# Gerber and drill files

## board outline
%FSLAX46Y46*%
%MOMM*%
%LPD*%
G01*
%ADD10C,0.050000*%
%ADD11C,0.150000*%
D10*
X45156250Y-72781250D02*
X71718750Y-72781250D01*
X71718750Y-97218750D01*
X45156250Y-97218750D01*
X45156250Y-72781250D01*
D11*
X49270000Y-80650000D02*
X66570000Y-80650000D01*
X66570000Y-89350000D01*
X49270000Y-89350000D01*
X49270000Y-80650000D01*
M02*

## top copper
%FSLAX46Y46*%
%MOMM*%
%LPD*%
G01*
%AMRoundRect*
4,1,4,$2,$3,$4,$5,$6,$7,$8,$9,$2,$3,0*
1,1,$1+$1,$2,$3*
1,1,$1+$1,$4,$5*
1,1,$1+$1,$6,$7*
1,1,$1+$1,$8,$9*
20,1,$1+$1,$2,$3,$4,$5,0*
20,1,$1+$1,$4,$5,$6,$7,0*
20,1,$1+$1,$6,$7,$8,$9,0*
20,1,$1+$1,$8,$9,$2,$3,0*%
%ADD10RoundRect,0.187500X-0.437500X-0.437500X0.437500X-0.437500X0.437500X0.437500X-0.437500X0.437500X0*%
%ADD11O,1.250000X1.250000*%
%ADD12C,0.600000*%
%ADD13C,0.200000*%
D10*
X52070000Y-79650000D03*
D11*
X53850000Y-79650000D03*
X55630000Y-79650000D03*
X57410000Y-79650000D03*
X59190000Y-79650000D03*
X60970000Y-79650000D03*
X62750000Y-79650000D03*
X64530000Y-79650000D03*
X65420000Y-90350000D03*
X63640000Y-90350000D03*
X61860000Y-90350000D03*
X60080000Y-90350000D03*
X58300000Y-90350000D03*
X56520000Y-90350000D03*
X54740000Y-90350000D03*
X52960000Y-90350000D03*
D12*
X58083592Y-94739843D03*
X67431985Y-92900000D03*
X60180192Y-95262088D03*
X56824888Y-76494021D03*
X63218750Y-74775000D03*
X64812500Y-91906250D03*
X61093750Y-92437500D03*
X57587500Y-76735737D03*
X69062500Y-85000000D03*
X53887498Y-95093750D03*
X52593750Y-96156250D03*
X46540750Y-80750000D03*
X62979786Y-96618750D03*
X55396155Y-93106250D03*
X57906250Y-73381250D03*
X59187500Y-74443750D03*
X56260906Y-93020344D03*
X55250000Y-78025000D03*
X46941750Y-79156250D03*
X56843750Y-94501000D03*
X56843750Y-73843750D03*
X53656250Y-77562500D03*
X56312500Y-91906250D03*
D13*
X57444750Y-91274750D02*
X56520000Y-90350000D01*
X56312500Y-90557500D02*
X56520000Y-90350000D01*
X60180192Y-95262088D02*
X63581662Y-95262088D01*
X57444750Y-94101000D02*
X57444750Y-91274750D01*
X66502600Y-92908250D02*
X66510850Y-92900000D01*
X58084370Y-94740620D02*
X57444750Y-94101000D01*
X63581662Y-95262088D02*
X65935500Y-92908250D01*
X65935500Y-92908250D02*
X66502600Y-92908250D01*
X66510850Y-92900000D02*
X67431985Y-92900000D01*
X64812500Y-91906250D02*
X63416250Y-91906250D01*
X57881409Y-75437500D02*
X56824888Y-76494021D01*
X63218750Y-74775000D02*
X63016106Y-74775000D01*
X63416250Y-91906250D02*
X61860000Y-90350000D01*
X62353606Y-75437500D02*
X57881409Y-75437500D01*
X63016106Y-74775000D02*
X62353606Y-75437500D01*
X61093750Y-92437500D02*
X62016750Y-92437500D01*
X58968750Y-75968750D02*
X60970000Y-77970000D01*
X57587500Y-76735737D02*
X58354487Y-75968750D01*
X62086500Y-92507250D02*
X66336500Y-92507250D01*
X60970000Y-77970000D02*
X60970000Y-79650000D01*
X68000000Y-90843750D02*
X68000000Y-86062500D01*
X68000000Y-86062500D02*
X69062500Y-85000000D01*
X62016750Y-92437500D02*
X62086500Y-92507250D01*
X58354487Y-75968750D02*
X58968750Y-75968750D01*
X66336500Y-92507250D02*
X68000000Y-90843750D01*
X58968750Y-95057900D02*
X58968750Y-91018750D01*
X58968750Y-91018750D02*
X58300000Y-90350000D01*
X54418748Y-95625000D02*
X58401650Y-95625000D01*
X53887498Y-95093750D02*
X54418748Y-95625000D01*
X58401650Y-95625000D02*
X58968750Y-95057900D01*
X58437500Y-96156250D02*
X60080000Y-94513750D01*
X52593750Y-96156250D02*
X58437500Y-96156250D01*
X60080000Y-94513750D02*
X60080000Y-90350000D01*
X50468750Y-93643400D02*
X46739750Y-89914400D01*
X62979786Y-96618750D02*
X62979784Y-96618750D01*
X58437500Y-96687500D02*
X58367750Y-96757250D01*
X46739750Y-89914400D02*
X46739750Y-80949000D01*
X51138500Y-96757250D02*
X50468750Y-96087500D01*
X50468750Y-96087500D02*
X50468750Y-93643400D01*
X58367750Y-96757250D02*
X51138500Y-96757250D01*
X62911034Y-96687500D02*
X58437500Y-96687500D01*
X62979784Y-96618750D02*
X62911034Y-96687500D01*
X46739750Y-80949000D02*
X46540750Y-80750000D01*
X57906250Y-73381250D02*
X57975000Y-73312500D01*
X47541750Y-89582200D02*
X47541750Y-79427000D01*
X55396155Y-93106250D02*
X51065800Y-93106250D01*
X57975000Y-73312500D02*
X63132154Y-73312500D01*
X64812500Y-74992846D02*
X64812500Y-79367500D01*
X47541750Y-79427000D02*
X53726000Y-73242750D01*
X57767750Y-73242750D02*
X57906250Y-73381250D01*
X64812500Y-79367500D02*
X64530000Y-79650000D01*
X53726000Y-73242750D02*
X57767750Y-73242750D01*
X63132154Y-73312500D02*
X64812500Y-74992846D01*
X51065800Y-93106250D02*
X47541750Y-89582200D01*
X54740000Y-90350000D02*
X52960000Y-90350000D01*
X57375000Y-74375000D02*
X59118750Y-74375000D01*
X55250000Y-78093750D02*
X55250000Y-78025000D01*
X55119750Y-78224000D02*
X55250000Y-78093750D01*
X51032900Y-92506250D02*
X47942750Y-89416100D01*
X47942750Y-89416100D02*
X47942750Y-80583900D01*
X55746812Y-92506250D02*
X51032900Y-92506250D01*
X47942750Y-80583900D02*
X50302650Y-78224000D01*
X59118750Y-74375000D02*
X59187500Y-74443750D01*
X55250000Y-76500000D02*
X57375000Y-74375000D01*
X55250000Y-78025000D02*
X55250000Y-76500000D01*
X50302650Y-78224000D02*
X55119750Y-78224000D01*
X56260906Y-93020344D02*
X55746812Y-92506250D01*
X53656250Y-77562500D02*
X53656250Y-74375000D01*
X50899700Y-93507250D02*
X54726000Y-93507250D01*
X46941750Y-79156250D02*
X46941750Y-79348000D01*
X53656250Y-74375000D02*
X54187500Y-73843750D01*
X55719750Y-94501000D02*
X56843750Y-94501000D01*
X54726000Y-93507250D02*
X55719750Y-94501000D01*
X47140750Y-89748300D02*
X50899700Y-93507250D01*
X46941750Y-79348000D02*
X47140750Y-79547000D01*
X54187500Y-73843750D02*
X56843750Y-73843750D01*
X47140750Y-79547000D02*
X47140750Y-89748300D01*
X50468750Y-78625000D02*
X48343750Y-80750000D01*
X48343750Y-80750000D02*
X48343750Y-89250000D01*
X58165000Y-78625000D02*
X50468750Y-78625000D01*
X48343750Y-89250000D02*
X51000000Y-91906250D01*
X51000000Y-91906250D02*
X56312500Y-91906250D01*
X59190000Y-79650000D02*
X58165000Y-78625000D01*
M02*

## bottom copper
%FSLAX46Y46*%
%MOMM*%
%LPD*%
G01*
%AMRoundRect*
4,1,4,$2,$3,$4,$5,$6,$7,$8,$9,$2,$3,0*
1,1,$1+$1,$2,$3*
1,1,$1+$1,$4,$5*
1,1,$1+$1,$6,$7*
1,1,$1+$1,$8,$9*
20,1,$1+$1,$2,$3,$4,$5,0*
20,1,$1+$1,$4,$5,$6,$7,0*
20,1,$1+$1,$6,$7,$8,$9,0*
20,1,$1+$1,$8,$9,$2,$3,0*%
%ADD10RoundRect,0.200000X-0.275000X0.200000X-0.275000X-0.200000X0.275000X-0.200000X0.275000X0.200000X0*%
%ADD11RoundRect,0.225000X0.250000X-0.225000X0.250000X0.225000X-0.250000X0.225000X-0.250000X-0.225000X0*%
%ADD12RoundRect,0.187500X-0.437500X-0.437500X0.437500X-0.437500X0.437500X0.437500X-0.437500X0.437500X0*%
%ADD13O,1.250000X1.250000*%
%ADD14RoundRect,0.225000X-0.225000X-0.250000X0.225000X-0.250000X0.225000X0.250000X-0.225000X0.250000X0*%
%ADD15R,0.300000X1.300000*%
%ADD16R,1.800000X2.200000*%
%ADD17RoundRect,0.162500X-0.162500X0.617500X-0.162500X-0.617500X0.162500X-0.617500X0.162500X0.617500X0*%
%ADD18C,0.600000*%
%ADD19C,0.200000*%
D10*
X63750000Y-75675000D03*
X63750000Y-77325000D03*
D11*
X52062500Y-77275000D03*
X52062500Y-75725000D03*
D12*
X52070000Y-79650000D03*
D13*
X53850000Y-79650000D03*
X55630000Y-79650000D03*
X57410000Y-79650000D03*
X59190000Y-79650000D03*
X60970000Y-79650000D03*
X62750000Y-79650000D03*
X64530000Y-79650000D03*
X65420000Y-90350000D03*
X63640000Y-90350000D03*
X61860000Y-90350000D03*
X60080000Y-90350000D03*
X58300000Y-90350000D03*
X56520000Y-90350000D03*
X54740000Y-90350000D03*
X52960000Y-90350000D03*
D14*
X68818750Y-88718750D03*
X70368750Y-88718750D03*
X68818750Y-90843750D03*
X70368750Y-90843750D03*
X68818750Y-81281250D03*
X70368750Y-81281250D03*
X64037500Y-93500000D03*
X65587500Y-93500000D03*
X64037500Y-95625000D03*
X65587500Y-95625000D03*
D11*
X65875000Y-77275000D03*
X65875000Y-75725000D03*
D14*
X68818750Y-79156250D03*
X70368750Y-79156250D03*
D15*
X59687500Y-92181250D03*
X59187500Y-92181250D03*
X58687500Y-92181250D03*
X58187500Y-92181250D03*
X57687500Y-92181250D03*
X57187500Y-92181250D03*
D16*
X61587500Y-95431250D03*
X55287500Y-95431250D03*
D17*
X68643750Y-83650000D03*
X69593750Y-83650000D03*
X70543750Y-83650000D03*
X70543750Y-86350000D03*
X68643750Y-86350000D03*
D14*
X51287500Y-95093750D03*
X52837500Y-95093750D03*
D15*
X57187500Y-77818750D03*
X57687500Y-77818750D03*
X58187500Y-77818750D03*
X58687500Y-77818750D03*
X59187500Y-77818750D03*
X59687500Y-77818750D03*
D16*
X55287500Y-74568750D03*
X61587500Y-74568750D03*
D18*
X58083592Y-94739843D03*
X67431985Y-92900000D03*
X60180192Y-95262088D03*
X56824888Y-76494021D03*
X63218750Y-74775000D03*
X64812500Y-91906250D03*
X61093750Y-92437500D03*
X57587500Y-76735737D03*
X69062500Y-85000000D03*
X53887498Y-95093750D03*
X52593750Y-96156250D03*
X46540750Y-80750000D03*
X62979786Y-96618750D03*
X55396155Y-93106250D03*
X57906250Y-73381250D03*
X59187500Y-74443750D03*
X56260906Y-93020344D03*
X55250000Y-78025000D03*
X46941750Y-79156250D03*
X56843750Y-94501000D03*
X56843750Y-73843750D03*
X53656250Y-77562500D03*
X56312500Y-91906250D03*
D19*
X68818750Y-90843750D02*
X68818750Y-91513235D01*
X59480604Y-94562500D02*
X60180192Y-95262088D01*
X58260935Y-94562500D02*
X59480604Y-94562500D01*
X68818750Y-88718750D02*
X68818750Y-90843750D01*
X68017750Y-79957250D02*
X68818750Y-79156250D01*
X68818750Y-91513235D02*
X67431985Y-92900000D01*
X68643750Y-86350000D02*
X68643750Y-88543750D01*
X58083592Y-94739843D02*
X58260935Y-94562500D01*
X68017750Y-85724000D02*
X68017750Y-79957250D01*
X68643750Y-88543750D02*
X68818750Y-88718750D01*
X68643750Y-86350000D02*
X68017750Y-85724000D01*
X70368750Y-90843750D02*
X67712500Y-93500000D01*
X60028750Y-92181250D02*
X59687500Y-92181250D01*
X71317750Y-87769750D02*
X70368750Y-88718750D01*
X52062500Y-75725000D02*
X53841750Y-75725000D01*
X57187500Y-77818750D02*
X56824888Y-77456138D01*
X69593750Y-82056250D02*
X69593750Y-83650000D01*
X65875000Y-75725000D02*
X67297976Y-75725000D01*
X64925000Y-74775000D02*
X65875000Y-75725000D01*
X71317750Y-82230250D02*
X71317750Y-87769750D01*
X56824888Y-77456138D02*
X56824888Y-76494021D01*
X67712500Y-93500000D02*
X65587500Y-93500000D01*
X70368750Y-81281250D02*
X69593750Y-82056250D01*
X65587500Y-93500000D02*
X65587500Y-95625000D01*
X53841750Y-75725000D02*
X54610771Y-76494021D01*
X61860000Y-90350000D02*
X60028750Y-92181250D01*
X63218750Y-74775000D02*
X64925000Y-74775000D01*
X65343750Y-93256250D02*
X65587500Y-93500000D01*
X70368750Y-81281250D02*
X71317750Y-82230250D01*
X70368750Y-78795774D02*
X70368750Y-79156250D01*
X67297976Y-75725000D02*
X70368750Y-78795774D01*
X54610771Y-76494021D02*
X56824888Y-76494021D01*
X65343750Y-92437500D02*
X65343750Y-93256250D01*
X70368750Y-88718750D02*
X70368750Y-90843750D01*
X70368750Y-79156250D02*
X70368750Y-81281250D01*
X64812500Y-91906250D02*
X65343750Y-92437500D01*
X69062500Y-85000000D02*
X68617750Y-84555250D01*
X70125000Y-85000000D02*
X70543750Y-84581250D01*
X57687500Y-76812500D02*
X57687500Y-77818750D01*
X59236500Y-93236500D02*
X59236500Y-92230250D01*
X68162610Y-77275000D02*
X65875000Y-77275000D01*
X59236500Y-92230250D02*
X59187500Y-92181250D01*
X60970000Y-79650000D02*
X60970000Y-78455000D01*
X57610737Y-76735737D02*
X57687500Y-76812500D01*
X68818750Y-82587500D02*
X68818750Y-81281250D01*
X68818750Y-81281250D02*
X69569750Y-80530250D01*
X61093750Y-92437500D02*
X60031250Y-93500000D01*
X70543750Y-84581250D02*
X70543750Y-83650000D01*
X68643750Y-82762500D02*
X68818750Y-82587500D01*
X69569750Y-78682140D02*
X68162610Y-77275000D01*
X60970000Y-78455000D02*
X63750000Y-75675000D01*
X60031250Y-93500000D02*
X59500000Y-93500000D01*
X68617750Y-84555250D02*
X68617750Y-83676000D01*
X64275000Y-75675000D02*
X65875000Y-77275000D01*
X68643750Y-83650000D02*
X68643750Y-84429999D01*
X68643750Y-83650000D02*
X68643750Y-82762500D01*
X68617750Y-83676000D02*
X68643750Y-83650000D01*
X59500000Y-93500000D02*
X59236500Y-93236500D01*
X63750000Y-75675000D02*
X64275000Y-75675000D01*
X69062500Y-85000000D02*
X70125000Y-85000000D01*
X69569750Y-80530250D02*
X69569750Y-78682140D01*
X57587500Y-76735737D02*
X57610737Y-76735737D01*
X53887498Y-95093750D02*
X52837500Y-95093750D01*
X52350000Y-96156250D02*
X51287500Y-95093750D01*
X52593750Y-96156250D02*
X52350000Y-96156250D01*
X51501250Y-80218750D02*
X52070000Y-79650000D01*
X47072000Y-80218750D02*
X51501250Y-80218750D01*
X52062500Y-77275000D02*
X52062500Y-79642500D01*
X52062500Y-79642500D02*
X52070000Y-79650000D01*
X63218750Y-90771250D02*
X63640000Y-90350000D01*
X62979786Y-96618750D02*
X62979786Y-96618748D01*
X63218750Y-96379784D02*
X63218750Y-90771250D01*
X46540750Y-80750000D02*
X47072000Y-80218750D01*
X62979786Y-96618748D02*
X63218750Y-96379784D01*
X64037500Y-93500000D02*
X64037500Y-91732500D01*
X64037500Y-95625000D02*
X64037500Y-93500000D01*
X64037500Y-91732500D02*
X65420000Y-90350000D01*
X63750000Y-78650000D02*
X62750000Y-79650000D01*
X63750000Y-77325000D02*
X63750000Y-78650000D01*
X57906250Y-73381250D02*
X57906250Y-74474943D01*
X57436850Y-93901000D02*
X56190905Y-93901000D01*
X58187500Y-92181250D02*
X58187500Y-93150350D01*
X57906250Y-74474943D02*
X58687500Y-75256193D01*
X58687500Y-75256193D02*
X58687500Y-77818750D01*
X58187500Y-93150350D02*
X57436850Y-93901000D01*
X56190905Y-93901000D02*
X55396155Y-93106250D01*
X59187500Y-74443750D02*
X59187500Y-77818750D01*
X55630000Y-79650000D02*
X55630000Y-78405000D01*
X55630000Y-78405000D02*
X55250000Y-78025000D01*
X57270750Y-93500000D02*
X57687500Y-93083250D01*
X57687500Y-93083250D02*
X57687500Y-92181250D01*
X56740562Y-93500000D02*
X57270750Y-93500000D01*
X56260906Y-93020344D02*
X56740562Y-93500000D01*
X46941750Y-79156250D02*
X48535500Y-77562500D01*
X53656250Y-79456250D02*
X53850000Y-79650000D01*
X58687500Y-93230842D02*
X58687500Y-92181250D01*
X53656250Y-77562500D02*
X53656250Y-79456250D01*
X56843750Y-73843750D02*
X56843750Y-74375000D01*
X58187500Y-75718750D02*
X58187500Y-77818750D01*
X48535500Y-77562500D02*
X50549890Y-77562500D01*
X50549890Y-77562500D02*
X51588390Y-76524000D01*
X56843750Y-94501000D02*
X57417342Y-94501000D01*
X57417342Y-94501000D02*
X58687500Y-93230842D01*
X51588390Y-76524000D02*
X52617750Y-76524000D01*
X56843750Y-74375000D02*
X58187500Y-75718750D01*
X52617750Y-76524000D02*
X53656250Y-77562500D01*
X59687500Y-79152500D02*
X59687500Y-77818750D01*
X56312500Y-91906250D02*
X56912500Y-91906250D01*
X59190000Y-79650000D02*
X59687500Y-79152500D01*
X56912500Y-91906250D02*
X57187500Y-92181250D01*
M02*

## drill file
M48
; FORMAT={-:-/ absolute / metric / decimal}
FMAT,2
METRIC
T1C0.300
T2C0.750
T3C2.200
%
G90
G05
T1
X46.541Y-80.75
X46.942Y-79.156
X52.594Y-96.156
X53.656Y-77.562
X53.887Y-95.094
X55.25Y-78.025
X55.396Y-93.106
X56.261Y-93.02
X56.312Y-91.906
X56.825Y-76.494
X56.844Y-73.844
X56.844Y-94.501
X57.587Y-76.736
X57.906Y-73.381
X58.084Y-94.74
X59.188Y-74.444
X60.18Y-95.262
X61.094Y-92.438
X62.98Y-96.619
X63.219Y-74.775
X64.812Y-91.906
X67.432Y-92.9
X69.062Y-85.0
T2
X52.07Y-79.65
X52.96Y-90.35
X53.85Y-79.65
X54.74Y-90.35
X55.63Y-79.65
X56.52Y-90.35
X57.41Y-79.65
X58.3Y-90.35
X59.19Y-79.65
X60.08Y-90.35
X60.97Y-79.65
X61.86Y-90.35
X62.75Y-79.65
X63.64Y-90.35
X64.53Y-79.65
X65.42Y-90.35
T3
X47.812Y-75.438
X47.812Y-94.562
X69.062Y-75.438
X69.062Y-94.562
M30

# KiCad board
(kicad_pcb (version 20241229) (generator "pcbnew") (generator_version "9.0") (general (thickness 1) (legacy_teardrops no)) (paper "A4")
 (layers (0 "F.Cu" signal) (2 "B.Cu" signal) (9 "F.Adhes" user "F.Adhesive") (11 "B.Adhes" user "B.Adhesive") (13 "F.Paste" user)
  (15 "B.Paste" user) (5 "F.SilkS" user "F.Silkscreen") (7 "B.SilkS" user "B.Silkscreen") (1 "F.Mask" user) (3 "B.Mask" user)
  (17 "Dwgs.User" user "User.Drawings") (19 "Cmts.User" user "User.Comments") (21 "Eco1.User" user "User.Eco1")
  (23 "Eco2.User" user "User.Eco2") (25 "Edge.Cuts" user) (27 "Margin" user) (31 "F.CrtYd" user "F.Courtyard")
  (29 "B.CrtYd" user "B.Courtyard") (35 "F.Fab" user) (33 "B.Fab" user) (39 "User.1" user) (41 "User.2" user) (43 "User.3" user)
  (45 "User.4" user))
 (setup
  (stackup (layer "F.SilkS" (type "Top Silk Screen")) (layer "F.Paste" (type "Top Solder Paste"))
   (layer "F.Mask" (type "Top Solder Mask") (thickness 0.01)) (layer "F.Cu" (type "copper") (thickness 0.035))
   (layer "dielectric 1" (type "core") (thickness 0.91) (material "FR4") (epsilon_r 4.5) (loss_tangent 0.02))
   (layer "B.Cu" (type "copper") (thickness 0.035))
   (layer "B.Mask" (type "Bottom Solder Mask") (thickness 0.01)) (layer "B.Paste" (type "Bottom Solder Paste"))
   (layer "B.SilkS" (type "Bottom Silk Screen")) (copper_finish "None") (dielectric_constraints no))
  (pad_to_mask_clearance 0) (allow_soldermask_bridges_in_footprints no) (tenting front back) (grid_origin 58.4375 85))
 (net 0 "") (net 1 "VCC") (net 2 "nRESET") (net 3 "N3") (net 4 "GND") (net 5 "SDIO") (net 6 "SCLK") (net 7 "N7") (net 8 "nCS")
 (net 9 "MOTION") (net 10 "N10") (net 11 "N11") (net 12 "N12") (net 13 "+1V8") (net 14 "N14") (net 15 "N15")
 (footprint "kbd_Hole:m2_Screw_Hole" (layer "F.Cu") (at 69.0625 75.4375)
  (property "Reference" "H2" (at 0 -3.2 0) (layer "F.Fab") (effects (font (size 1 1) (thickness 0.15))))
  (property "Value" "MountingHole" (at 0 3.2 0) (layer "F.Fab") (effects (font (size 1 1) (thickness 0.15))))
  (pad "" np_thru_hole circle (at 0 0) (size 2.2 2.2) (drill 2.2) (layers "*.Cu" "*.Mask")))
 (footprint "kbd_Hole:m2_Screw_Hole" (layer "F.Cu") (at 47.8125 94.5625)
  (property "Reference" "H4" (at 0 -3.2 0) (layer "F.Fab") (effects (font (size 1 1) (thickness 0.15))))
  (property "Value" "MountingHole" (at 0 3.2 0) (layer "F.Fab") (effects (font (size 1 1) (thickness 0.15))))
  (pad "" np_thru_hole circle (at 0 0) (size 2.2 2.2) (drill 2.2) (layers "*.Cu" "*.Mask")))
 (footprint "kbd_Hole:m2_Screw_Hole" (layer "F.Cu") (at 47.8125 75.4375)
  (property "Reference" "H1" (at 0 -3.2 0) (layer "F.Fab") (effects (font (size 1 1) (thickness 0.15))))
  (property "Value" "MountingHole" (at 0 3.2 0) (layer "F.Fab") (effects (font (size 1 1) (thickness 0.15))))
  (pad "" np_thru_hole circle (at 0 0) (size 2.2 2.2) (drill 2.2) (layers "*.Cu" "*.Mask")))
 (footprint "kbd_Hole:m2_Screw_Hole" (layer "F.Cu") (at 69.0625 94.5625)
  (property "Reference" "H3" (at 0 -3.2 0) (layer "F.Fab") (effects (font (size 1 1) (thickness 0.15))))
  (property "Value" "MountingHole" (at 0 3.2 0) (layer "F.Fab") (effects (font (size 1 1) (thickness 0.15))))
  (pad "" np_thru_hole circle (at 0 0) (size 2.2 2.2) (drill 2.2) (layers "*.Cu" "*.Mask")))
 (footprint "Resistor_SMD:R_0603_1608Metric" (layer "B.Cu") (at 63.75 76.5 -90)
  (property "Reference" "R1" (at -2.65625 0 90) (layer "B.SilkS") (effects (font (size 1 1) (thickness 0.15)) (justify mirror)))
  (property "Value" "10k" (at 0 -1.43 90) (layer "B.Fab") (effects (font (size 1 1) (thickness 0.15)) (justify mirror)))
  (pad "1" smd roundrect (at -0.825 0 270) (size 0.8 0.95) (layers "B.Cu" "B.Mask" "B.Paste") (roundrect_rratio 0.25) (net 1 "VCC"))
  (pad "2" smd roundrect (at 0.825 0 270) (size 0.8 0.95) (layers "B.Cu" "B.Mask" "B.Paste") (roundrect_rratio 0.25) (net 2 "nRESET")))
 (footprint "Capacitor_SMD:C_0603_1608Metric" (layer "B.Cu") (at 52.0625 76.5 90)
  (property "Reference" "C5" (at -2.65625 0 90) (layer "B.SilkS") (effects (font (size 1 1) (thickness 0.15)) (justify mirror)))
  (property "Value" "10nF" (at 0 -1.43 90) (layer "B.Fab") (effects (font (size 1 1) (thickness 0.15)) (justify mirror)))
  (pad "1" smd roundrect (at -0.775 0 90) (size 0.9 0.95) (layers "B.Cu" "B.Mask" "B.Paste") (roundrect_rratio 0.25) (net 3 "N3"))
  (pad "2" smd roundrect (at 0.775 0 90) (size 0.9 0.95) (layers "B.Cu" "B.Mask" "B.Paste") (roundrect_rratio 0.25) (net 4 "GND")))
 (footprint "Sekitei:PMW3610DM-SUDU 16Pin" (layer "B.Cu") (at 58.238 85 180)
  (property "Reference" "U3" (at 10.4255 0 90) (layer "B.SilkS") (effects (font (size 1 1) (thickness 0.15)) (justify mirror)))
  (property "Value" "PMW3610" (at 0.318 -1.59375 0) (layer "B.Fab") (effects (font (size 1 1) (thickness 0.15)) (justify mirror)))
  (fp_rect (start 8.968 4.35) (end -8.332 -4.35) (stroke (width 0.15) (type solid)) (fill no) (layer "Edge.Cuts"))
  (pad "1" thru_hole roundrect (at 6.168 5.35) (size 1.25 1.25) (drill 0.75) (layers "*.Cu" "*.Mask") (remove_unused_layers no)
   (roundrect_rratio 0.15) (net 3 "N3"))
  (pad "2" thru_hole oval (at 4.388 5.35) (size 1.25 1.25) (drill 0.75) (layers "*.Cu" "*.Mask") (remove_unused_layers no) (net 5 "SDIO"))
  (pad "3" thru_hole oval (at 2.608 5.35) (size 1.25 1.25) (drill 0.75) (layers "*.Cu" "*.Mask") (remove_unused_layers no) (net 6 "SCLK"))
  (pad "4" thru_hole oval (at 0.828 5.35) (size 1.25 1.25) (drill 0.75) (layers "*.Cu" "*.Mask") (remove_unused_layers no) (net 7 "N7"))
  (pad "5" thru_hole oval (at -0.952 5.35) (size 1.25 1.25) (drill 0.75) (layers "*.Cu" "*.Mask") (remove_unused_layers no) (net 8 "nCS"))
  (pad "6" thru_hole oval (at -2.732 5.35) (size 1.25 1.25) (drill 0.75) (layers "*.Cu" "*.Mask") (remove_unused_layers no) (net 1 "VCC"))
  (pad "7" thru_hole oval (at -4.512 5.35) (size 1.25 1.25) (drill 0.75) (layers "*.Cu" "*.Mask") (remove_unused_layers no) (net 2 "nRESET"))
  (pad "8" thru_hole oval (at -6.292 5.35) (size 1.25 1.25) (drill 0.75) (layers "*.Cu" "*.Mask") (remove_unused_layers no) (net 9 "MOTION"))
  (pad "9" thru_hole oval (at -7.182 -5.35) (size 1.25 1.25) (drill 0.75) (layers "*.Cu" "*.Mask") (remove_unused_layers no) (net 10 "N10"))
  (pad "10" thru_hole oval (at -5.402 -5.35) (size 1.25 1.25) (drill 0.75) (layers "*.Cu" "*.Mask") (remove_unused_layers no) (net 3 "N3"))
  (pad "11" thru_hole oval (at -3.622 -5.35) (size 1.25 1.25) (drill 0.75) (layers "*.Cu" "*.Mask") (remove_unused_layers no) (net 4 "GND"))
  (pad "12" thru_hole oval (at -1.842 -5.35) (size 1.25 1.25) (drill 0.75) (layers "*.Cu" "*.Mask") (remove_unused_layers no) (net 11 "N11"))
  (pad "13" thru_hole oval (at -0.062 -5.35) (size 1.25 1.25) (drill 0.75) (layers "*.Cu" "*.Mask") (remove_unused_layers no) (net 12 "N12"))
  (pad "14" thru_hole oval (at 1.718 -5.35) (size 1.25 1.25) (drill 0.75) (layers "*.Cu" "*.Mask") (remove_unused_layers no) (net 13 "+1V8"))
  (pad "15" thru_hole oval (at 3.498 -5.35) (size 1.25 1.25) (drill 0.75) (layers "*.Cu" "*.Mask") (remove_unused_layers no) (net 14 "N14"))
  (pad "16" thru_hole oval (at 5.278 -5.35) (size 1.25 1.25) (drill 0.75) (layers "*.Cu" "*.Mask") (remove_unused_layers no) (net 14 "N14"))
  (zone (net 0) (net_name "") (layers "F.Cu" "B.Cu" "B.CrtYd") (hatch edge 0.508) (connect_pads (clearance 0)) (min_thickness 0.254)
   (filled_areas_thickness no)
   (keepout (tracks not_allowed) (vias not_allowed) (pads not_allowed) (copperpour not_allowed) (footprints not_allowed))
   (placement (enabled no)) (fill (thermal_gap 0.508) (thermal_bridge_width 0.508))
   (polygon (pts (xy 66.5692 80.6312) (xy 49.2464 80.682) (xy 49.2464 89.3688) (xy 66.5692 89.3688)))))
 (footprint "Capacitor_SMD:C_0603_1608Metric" (layer "B.Cu") (at 69.59375 88.71875)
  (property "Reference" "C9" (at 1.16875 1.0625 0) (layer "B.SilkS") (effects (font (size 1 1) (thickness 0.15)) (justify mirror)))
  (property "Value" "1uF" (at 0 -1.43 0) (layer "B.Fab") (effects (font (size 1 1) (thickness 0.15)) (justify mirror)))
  (pad "1" smd roundrect (at -0.775 0) (size 0.9 0.95) (layers "B.Cu" "B.Mask" "B.Paste") (roundrect_rratio 0.25) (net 13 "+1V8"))
  (pad "2" smd roundrect (at 0.775 0) (size 0.9 0.95) (layers "B.Cu" "B.Mask" "B.Paste") (roundrect_rratio 0.25) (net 4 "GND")))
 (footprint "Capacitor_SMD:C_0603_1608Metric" (layer "B.Cu") (at 69.59375 90.84375)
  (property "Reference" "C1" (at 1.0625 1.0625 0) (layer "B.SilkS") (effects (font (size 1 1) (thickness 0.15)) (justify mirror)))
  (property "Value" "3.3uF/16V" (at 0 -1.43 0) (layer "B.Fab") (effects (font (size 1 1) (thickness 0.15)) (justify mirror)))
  (pad "1" smd roundrect (at -0.775 0) (size 0.9 0.95) (layers "B.Cu" "B.Mask" "B.Paste") (roundrect_rratio 0.25) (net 13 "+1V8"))
  (pad "2" smd roundrect (at 0.775 0) (size 0.9 0.95) (layers "B.Cu" "B.Mask" "B.Paste") (roundrect_rratio 0.25) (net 4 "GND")))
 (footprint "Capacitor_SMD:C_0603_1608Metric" (layer "B.Cu") (at 69.59375 81.28125)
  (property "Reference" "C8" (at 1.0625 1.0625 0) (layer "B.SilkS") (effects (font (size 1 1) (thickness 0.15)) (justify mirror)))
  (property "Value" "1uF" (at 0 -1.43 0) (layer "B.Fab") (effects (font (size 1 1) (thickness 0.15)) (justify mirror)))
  (pad "1" smd roundrect (at -0.775 0) (size 0.9 0.95) (layers "B.Cu" "B.Mask" "B.Paste") (roundrect_rratio 0.25) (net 1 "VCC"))
  (pad "2" smd roundrect (at 0.775 0) (size 0.9 0.95) (layers "B.Cu" "B.Mask" "B.Paste") (roundrect_rratio 0.25) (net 4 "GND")))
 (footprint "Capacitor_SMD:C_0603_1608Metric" (layer "B.Cu") (at 64.8125 93.5)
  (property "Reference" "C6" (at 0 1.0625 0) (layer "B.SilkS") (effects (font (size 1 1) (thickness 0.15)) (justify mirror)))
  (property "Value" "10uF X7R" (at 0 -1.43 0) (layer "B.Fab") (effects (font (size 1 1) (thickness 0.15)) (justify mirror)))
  (pad "1" smd roundrect (at -0.775 0) (size 0.9 0.95) (layers "B.Cu" "B.Mask" "B.Paste") (roundrect_rratio 0.25) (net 10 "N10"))
  (pad "2" smd roundrect (at 0.775 0) (size 0.9 0.95) (layers "B.Cu" "B.Mask" "B.Paste") (roundrect_rratio 0.25) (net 4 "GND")))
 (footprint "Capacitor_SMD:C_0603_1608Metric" (layer "B.Cu") (at 64.8125 95.625)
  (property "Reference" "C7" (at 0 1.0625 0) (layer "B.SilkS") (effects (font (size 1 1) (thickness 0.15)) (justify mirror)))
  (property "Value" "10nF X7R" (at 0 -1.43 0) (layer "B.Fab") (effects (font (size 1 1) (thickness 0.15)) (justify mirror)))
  (pad "1" smd roundrect (at -0.775 0) (size 0.9 0.95) (layers "B.Cu" "B.Mask" "B.Paste") (roundrect_rratio 0.25) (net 10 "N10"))
  (pad "2" smd roundrect (at 0.775 0) (size 0.9 0.95) (layers "B.Cu" "B.Mask" "B.Paste") (roundrect_rratio 0.25) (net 4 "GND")))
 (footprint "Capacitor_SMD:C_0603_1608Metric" (layer "B.Cu") (at 65.875 76.5 90)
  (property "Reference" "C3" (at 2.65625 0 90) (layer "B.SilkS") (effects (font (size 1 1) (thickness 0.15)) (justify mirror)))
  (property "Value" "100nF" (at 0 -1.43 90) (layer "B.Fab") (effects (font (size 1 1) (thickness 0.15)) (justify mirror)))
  (pad "1" smd roundrect (at -0.775 0 90) (size 0.9 0.95) (layers "B.Cu" "B.Mask" "B.Paste") (roundrect_rratio 0.25) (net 1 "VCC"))
  (pad "2" smd roundrect (at 0.775 0 90) (size 0.9 0.95) (layers "B.Cu" "B.Mask" "B.Paste") (roundrect_rratio 0.25) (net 4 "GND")))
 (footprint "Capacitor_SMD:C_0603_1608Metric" (layer "B.Cu") (at 69.59375 79.15625)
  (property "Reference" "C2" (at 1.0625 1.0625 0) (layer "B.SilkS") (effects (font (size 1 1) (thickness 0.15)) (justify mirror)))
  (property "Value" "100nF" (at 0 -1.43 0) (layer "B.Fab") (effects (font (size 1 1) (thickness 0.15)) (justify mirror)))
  (pad "1" smd roundrect (at -0.775 0) (size 0.9 0.95) (layers "B.Cu" "B.Mask" "B.Paste") (roundrect_rratio 0.25) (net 13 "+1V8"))
  (pad "2" smd roundrect (at 0.775 0) (size 0.9 0.95) (layers "B.Cu" "B.Mask" "B.Paste") (roundrect_rratio 0.25) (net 4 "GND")))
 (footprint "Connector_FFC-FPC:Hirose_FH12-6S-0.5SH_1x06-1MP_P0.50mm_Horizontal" (layer "B.Cu") (at 58.4375 94.03125 180)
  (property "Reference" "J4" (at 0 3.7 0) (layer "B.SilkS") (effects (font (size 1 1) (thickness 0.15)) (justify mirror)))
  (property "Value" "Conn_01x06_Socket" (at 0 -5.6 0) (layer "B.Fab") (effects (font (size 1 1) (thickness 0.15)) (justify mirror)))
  (pad "1" smd rect (at -1.25 1.85 180) (size 0.3 1.3) (layers "B.Cu" "B.Mask" "B.Paste") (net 4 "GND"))
  (pad "2" smd rect (at -0.75 1.85 180) (size 0.3 1.3) (layers "B.Cu" "B.Mask" "B.Paste") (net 1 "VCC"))
  (pad "3" smd rect (at -0.25 1.85 180) (size 0.3 1.3) (layers "B.Cu" "B.Mask" "B.Paste") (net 5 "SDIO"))
  (pad "4" smd rect (at 0.25 1.85 180) (size 0.3 1.3) (layers "B.Cu" "B.Mask" "B.Paste") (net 9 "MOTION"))
  (pad "5" smd rect (at 0.75 1.85 180) (size 0.3 1.3) (layers "B.Cu" "B.Mask" "B.Paste") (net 6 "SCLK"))
  (pad "6" smd rect (at 1.25 1.85 180) (size 0.3 1.3) (layers "B.Cu" "B.Mask" "B.Paste") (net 8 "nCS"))
  (pad "MP" smd rect (at -3.15 -1.4 180) (size 1.8 2.2) (layers "B.Cu" "B.Mask" "B.Paste"))
  (pad "MP" smd rect (at 3.15 -1.4 180) (size 1.8 2.2) (layers "B.Cu" "B.Mask" "B.Paste")))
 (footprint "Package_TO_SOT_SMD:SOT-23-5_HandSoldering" (layer "B.Cu") (at 69.59375 85 -90)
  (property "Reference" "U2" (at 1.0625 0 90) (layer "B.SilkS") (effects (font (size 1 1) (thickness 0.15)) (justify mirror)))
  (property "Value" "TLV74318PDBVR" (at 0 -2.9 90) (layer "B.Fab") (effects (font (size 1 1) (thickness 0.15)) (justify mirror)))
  (pad "1" smd roundrect (at -1.35 0.95 270) (size 1.56 0.65) (layers "B.Cu" "B.Mask" "B.Paste") (roundrect_rratio 0.25) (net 1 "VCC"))
  (pad "2" smd roundrect (at -1.35 0 270) (size 1.56 0.65) (layers "B.Cu" "B.Mask" "B.Paste") (roundrect_rratio 0.25) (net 4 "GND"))
  (pad "3" smd roundrect (at -1.35 -0.95 270) (size 1.56 0.65) (layers "B.Cu" "B.Mask" "B.Paste") (roundrect_rratio 0.25) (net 1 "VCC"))
  (pad "4" smd roundrect (at 1.35 -0.95 270) (size 1.56 0.65) (layers "B.Cu" "B.Mask" "B.Paste") (roundrect_rratio 0.25) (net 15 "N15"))
  (pad "5" smd roundrect (at 1.35 0.95 270) (size 1.56 0.65) (layers "B.Cu" "B.Mask" "B.Paste") (roundrect_rratio 0.25) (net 13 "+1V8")))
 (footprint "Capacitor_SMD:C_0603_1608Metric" (layer "B.Cu") (at 52.0625 95.09375)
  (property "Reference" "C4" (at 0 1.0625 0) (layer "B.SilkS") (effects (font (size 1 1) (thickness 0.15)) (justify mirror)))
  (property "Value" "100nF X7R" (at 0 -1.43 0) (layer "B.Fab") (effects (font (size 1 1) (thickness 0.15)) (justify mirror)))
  (pad "1" smd roundrect (at -0.775 0) (size 0.9 0.95) (layers "B.Cu" "B.Mask" "B.Paste") (roundrect_rratio 0.25) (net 11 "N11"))
  (pad "2" smd roundrect (at 0.775 0) (size 0.9 0.95) (layers "B.Cu" "B.Mask" "B.Paste") (roundrect_rratio 0.25) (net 12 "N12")))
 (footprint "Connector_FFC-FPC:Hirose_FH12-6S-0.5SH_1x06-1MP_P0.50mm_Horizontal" (layer "B.Cu") (at 58.4375 75.96875)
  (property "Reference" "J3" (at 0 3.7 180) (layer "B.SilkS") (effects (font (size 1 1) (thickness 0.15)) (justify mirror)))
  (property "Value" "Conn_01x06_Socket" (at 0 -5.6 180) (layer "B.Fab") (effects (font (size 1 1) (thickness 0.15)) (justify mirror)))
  (pad "1" smd rect (at -1.25 1.85) (size 0.3 1.3) (layers "B.Cu" "B.Mask" "B.Paste") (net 4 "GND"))
  (pad "2" smd rect (at -0.75 1.85) (size 0.3 1.3) (layers "B.Cu" "B.Mask" "B.Paste") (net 1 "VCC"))
  (pad "3" smd rect (at -0.25 1.85) (size 0.3 1.3) (layers "B.Cu" "B.Mask" "B.Paste") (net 5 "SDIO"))
  (pad "4" smd rect (at 0.25 1.85) (size 0.3 1.3) (layers "B.Cu" "B.Mask" "B.Paste") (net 9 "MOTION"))
  (pad "5" smd rect (at 0.75 1.85) (size 0.3 1.3) (layers "B.Cu" "B.Mask" "B.Paste") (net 6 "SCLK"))
  (pad "6" smd rect (at 1.25 1.85) (size 0.3 1.3) (layers "B.Cu" "B.Mask" "B.Paste") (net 8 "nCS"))
  (pad "MP" smd rect (at -3.15 -1.4) (size 1.8 2.2) (layers "B.Cu" "B.Mask" "B.Paste"))
  (pad "MP" smd rect (at 3.15 -1.4) (size 1.8 2.2) (layers "B.Cu" "B.Mask" "B.Paste")))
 (gr_rect (start 45.15625 72.78125) (end 71.71875 97.21875) (stroke (width 0.05) (type default)) (fill no) (layer "Edge.Cuts"))
 (segment (start 57.44475 91.27475) (end 56.52 90.35) (width 0.2) (layer "F.Cu") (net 13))
 (segment (start 56.3125 90.5575) (end 56.52 90.35) (width 0.2) (layer "F.Cu") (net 13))
 (segment (start 60.180192 95.262088) (end 63.581662 95.262088) (width 0.2) (layer "F.Cu") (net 13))
 (segment (start 57.44475 94.101) (end 57.44475 91.27475) (width 0.2) (layer "F.Cu") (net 13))
 (segment (start 66.5026 92.90825) (end 66.51085 92.9) (width 0.2) (layer "F.Cu") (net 13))
 (segment (start 58.08437 94.74062) (end 57.44475 94.101) (width 0.2) (layer "F.Cu") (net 13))
 (segment (start 63.581662 95.262088) (end 65.9355 92.90825) (width 0.2) (layer "F.Cu") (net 13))
 (segment (start 65.9355 92.90825) (end 66.5026 92.90825) (width 0.2) (layer "F.Cu") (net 13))
 (segment (start 66.51085 92.9) (end 67.431985 92.9) (width 0.2) (layer "F.Cu") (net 13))
 (via (at 58.083592 94.739843) (size 0.6) (drill 0.3) (layers "F.Cu" "B.Cu") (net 13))
 (via (at 67.431985 92.9) (size 0.6) (drill 0.3) (layers "F.Cu" "B.Cu") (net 13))
 (via (at 60.180192 95.262088) (size 0.6) (drill 0.3) (layers "F.Cu" "B.Cu") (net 13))
 (segment (start 68.81875 90.84375) (end 68.81875 91.513235) (width 0.2) (layer "B.Cu") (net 13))
 (segment (start 59.480604 94.5625) (end 60.180192 95.262088) (width 0.2) (layer "B.Cu") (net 13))
 (segment (start 58.260935 94.5625) (end 59.480604 94.5625) (width 0.2) (layer "B.Cu") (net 13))
 (segment (start 68.81875 88.71875) (end 68.81875 90.84375) (width 0.2) (layer "B.Cu") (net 13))
 (segment (start 68.01775 79.95725) (end 68.81875 79.15625) (width 0.2) (layer "B.Cu") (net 13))
 (segment (start 68.81875 91.513235) (end 67.431985 92.9) (width 0.2) (layer "B.Cu") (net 13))
 (segment (start 68.64375 86.35) (end 68.64375 88.54375) (width 0.2) (layer "B.Cu") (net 13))
 (segment (start 58.083592 94.739843) (end 58.260935 94.5625) (width 0.2) (layer "B.Cu") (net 13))
 (segment (start 68.01775 85.724) (end 68.01775 79.95725) (width 0.2) (layer "B.Cu") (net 13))
 (segment (start 68.64375 88.54375) (end 68.81875 88.71875) (width 0.2) (layer "B.Cu") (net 13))
 (segment (start 68.64375 86.35) (end 68.01775 85.724) (width 0.2) (layer "B.Cu") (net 13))
 (segment (start 64.8125 91.90625) (end 63.41625 91.90625) (width 0.2) (layer "F.Cu") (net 4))
 (segment (start 57.881409 75.4375) (end 56.824888 76.494021) (width 0.2) (layer "F.Cu") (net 4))
 (segment (start 63.21875 74.775) (end 63.016106 74.775) (width 0.2) (layer "F.Cu") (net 4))
 (segment (start 63.41625 91.90625) (end 61.86 90.35) (width 0.2) (layer "F.Cu") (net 4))
 (segment (start 62.353606 75.4375) (end 57.881409 75.4375) (width 0.2) (layer "F.Cu") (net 4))
 (segment (start 63.016106 74.775) (end 62.353606 75.4375) (width 0.2) (layer "F.Cu") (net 4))
 (via (at 56.824888 76.494021) (size 0.6) (drill 0.3) (layers "F.Cu" "B.Cu") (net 4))
 (via (at 63.21875 74.775) (size 0.6) (drill 0.3) (layers "F.Cu" "B.Cu") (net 4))
 (via (at 64.8125 91.90625) (size 0.6) (drill 0.3) (layers "F.Cu" "B.Cu") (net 4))
 (segment (start 70.36875 90.84375) (end 67.7125 93.5) (width 0.2) (layer "B.Cu") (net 4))
 (segment (start 60.02875 92.18125) (end 59.6875 92.18125) (width 0.2) (layer "B.Cu") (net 4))
 (segment (start 71.31775 87.76975) (end 70.36875 88.71875) (width 0.2) (layer "B.Cu") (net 4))
 (segment (start 52.0625 75.725) (end 53.84175 75.725) (width 0.2) (layer "B.Cu") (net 4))
 (segment (start 57.1875 77.81875) (end 56.824888 77.456138) (width 0.2) (layer "B.Cu") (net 4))
 (segment (start 69.59375 82.05625) (end 69.59375 83.65) (width 0.2) (layer "B.Cu") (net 4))
 (segment (start 65.875 75.725) (end 67.297976 75.725) (width 0.2) (layer "B.Cu") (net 4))
 (segment (start 64.925 74.775) (end 65.875 75.725) (width 0.2) (layer "B.Cu") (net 4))
 (segment (start 71.31775 82.23025) (end 71.31775 87.76975) (width 0.2) (layer "B.Cu") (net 4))
 (segment (start 56.824888 77.456138) (end 56.824888 76.494021) (width 0.2) (layer "B.Cu") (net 4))
 (segment (start 67.7125 93.5) (end 65.5875 93.5) (width 0.2) (layer "B.Cu") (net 4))
 (segment (start 70.36875 81.28125) (end 69.59375 82.05625) (width 0.2) (layer "B.Cu") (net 4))
 (segment (start 65.5875 93.5) (end 65.5875 95.625) (width 0.2) (layer "B.Cu") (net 4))
 (segment (start 53.84175 75.725) (end 54.610771 76.494021) (width 0.2) (layer "B.Cu") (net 4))
 (segment (start 61.86 90.35) (end 60.02875 92.18125) (width 0.2) (layer "B.Cu") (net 4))
 (segment (start 63.21875 74.775) (end 64.925 74.775) (width 0.2) (layer "B.Cu") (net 4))
 (segment (start 65.34375 93.25625) (end 65.5875 93.5) (width 0.2) (layer "B.Cu") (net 4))
 (segment (start 70.36875 81.28125) (end 71.31775 82.23025) (width 0.2) (layer "B.Cu") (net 4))
 (segment (start 70.36875 78.795774) (end 70.36875 79.15625) (width 0.2) (layer "B.Cu") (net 4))
 (segment (start 67.297976 75.725) (end 70.36875 78.795774) (width 0.2) (layer "B.Cu") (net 4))
 (segment (start 54.610771 76.494021) (end 56.824888 76.494021) (width 0.2) (layer "B.Cu") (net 4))
 (segment (start 65.34375 92.4375) (end 65.34375 93.25625) (width 0.2) (layer "B.Cu") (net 4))
 (segment (start 70.36875 88.71875) (end 70.36875 90.84375) (width 0.2) (layer "B.Cu") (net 4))
 (segment (start 70.36875 79.15625) (end 70.36875 81.28125) (width 0.2) (layer "B.Cu") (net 4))
 (segment (start 64.8125 91.90625) (end 65.34375 92.4375) (width 0.2) (layer "B.Cu") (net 4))
 (segment (start 61.09375 92.4375) (end 62.01675 92.4375) (width 0.2) (layer "F.Cu") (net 1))
 (segment (start 58.96875 75.96875) (end 60.97 77.97) (width 0.2) (layer "F.Cu") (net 1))
 (segment (start 57.5875 76.735737) (end 58.354487 75.96875) (width 0.2) (layer "F.Cu") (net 1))
 (segment (start 62.0865 92.50725) (end 66.3365 92.50725) (width 0.2) (layer "F.Cu") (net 1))
 (segment (start 60.97 77.97) (end 60.97 79.65) (width 0.2) (layer "F.Cu") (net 1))
 (segment (start 68 90.84375) (end 68 86.0625) (width 0.2) (layer "F.Cu") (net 1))
 (segment (start 68 86.0625) (end 69.0625 85) (width 0.2) (layer "F.Cu") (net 1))
 (segment (start 62.01675 92.4375) (end 62.0865 92.50725) (width 0.2) (layer "F.Cu") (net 1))
 (segment (start 58.354487 75.96875) (end 58.96875 75.96875) (width 0.2) (layer "F.Cu") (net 1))
 (segment (start 66.3365 92.50725) (end 68 90.84375) (width 0.2) (layer "F.Cu") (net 1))
 (via (at 61.09375 92.4375) (size 0.6) (drill 0.3) (layers "F.Cu" "B.Cu") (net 1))
 (via (at 57.5875 76.735737) (size 0.6) (drill 0.3) (layers "F.Cu" "B.Cu") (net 1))
 (via (at 69.0625 85) (size 0.6) (drill 0.3) (layers "F.Cu" "B.Cu") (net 1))
 (segment (start 69.0625 85) (end 68.61775 84.55525) (width 0.2) (layer "B.Cu") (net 1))
 (segment (start 70.125 85) (end 70.54375 84.58125) (width 0.2) (layer "B.Cu") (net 1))
 (segment (start 57.6875 76.8125) (end 57.6875 77.81875) (width 0.2) (layer "B.Cu") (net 1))
 (segment (start 59.2365 93.2365) (end 59.2365 92.23025) (width 0.2) (layer "B.Cu") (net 1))
 (segment (start 68.16261 77.275) (end 65.875 77.275) (width 0.2) (layer "B.Cu") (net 1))
 (segment (start 59.2365 92.23025) (end 59.1875 92.18125) (width 0.2) (layer "B.Cu") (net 1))
 (segment (start 60.97 79.65) (end 60.97 78.455) (width 0.2) (layer "B.Cu") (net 1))
 (segment (start 57.610737 76.735737) (end 57.6875 76.8125) (width 0.2) (layer "B.Cu") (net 1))
 (segment (start 68.81875 82.5875) (end 68.81875 81.28125) (width 0.2) (layer "B.Cu") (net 1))
 (segment (start 68.81875 81.28125) (end 69.56975 80.53025) (width 0.2) (layer "B.Cu") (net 1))
 (segment (start 61.09375 92.4375) (end 60.03125 93.5) (width 0.2) (layer "B.Cu") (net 1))
 (segment (start 70.54375 84.58125) (end 70.54375 83.65) (width 0.2) (layer "B.Cu") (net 1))
 (segment (start 68.64375 82.7625) (end 68.81875 82.5875) (width 0.2) (layer "B.Cu") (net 1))
 (segment (start 69.56975 78.68214) (end 68.16261 77.275) (width 0.2) (layer "B.Cu") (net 1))
 (segment (start 60.97 78.455) (end 63.75 75.675) (width 0.2) (layer "B.Cu") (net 1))
 (segment (start 60.03125 93.5) (end 59.5 93.5) (width 0.2) (layer "B.Cu") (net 1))
 (segment (start 68.61775 84.55525) (end 68.61775 83.676) (width 0.2) (layer "B.Cu") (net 1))
 (segment (start 64.275 75.675) (end 65.875 77.275) (width 0.2) (layer "B.Cu") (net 1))
 (segment (start 68.64375 83.65) (end 68.64375 84.429999) (width 0.2) (layer "B.Cu") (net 1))
 (segment (start 68.64375 83.65) (end 68.64375 82.7625) (width 0.2) (layer "B.Cu") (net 1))
 (segment (start 68.61775 83.676) (end 68.64375 83.65) (width 0.2) (layer "B.Cu") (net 1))
 (segment (start 59.5 93.5) (end 59.2365 93.2365) (width 0.2) (layer "B.Cu") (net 1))
 (segment (start 63.75 75.675) (end 64.275 75.675) (width 0.2) (layer "B.Cu") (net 1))
 (segment (start 69.0625 85) (end 70.125 85) (width 0.2) (layer "B.Cu") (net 1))
 (segment (start 69.56975 80.53025) (end 69.56975 78.68214) (width 0.2) (layer "B.Cu") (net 1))
 (segment (start 57.5875 76.735737) (end 57.610737 76.735737) (width 0.2) (layer "B.Cu") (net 1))
 (segment (start 58.96875 95.0579) (end 58.96875 91.01875) (width 0.2) (layer "F.Cu") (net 12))
 (segment (start 58.96875 91.01875) (end 58.3 90.35) (width 0.2) (layer "F.Cu") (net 12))
 (segment (start 54.418748 95.625) (end 58.40165 95.625) (width 0.2) (layer "F.Cu") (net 12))
 (segment (start 53.887498 95.09375) (end 54.418748 95.625) (width 0.2) (layer "F.Cu") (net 12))
 (segment (start 58.40165 95.625) (end 58.96875 95.0579) (width 0.2) (layer "F.Cu") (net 12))
 (via (at 53.887498 95.09375) (size 0.6) (drill 0.3) (layers "F.Cu" "B.Cu") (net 12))
 (segment (start 53.887498 95.09375) (end 52.8375 95.09375) (width 0.2) (layer "B.Cu") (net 12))
 (segment (start 58.4375 96.15625) (end 60.08 94.51375) (width 0.2) (layer "F.Cu") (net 11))
 (segment (start 52.59375 96.15625) (end 58.4375 96.15625) (width 0.2) (layer "F.Cu") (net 11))
 (segment (start 60.08 94.51375) (end 60.08 90.35) (width 0.2) (layer "F.Cu") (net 11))
 (via (at 52.59375 96.15625) (size 0.6) (drill 0.3) (layers "F.Cu" "B.Cu") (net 11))
 (segment (start 52.35 96.15625) (end 51.2875 95.09375) (width 0.2) (layer "B.Cu") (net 11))
 (segment (start 52.59375 96.15625) (end 52.35 96.15625) (width 0.2) (layer "B.Cu") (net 11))
 (segment (start 50.46875 93.6434) (end 46.73975 89.9144) (width 0.2) (layer "F.Cu") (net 3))
 (segment (start 62.979786 96.61875) (end 62.979784 96.61875) (width 0.2) (layer "F.Cu") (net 3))
 (segment (start 58.4375 96.6875) (end 58.36775 96.75725) (width 0.2) (layer "F.Cu") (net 3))
 (segment (start 46.73975 89.9144) (end 46.73975 80.949) (width 0.2) (layer "F.Cu") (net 3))
 (segment (start 51.1385 96.75725) (end 50.46875 96.0875) (width 0.2) (layer "F.Cu") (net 3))
 (segment (start 50.46875 96.0875) (end 50.46875 93.6434) (width 0.2) (layer "F.Cu") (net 3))
 (segment (start 58.36775 96.75725) (end 51.1385 96.75725) (width 0.2) (layer "F.Cu") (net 3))
 (segment (start 62.911034 96.6875) (end 58.4375 96.6875) (width 0.2) (layer "F.Cu") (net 3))
 (segment (start 62.979784 96.61875) (end 62.911034 96.6875) (width 0.2) (layer "F.Cu") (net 3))
 (segment (start 46.73975 80.949) (end 46.54075 80.75) (width 0.2) (layer "F.Cu") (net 3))
 (via (at 46.54075 80.75) (size 0.6) (drill 0.3) (layers "F.Cu" "B.Cu") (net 3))
 (via (at 62.979786 96.61875) (size 0.6) (drill 0.3) (layers "F.Cu" "B.Cu") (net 3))
 (segment (start 51.50125 80.21875) (end 52.07 79.65) (width 0.2) (layer "B.Cu") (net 3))
 (segment (start 47.072 80.21875) (end 51.50125 80.21875) (width 0.2) (layer "B.Cu") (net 3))
 (segment (start 52.0625 77.275) (end 52.0625 79.6425) (width 0.2) (layer "B.Cu") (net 3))
 (segment (start 52.0625 79.6425) (end 52.07 79.65) (width 0.2) (layer "B.Cu") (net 3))
 (segment (start 63.21875 90.77125) (end 63.64 90.35) (width 0.2) (layer "B.Cu") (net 3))
 (segment (start 62.979786 96.61875) (end 62.979786 96.618748) (width 0.2) (layer "B.Cu") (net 3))
 (segment (start 63.21875 96.379784) (end 63.21875 90.77125) (width 0.2) (layer "B.Cu") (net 3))
 (segment (start 46.54075 80.75) (end 47.072 80.21875) (width 0.2) (layer "B.Cu") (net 3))
 (segment (start 62.979786 96.618748) (end 63.21875 96.379784) (width 0.2) (layer "B.Cu") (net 3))
 (segment (start 64.0375 93.5) (end 64.0375 91.7325) (width 0.2) (layer "B.Cu") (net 10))
 (segment (start 64.0375 95.625) (end 64.0375 93.5) (width 0.2) (layer "B.Cu") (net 10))
 (segment (start 64.0375 91.7325) (end 65.42 90.35) (width 0.2) (layer "B.Cu") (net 10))
 (segment (start 63.75 78.65) (end 62.75 79.65) (width 0.2) (layer "B.Cu") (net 2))
 (segment (start 63.75 77.325) (end 63.75 78.65) (width 0.2) (layer "B.Cu") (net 2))
 (segment (start 57.90625 73.38125) (end 57.975 73.3125) (width 0.2) (layer "F.Cu") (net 9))
 (segment (start 47.54175 89.5822) (end 47.54175 79.427) (width 0.2) (layer "F.Cu") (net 9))
 (segment (start 55.396155 93.10625) (end 51.0658 93.10625) (width 0.2) (layer "F.Cu") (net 9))
 (segment (start 57.975 73.3125) (end 63.132154 73.3125) (width 0.2) (layer "F.Cu") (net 9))
 (segment (start 64.8125 74.992846) (end 64.8125 79.3675) (width 0.2) (layer "F.Cu") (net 9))
 (segment (start 47.54175 79.427) (end 53.726 73.24275) (width 0.2) (layer "F.Cu") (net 9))
 (segment (start 57.76775 73.24275) (end 57.90625 73.38125) (width 0.2) (layer "F.Cu") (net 9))
 (segment (start 64.8125 79.3675) (end 64.53 79.65) (width 0.2) (layer "F.Cu") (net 9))
 (segment (start 53.726 73.24275) (end 57.76775 73.24275) (width 0.2) (layer "F.Cu") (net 9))
 (segment (start 63.132154 73.3125) (end 64.8125 74.992846) (width 0.2) (layer "F.Cu") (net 9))
 (segment (start 51.0658 93.10625) (end 47.54175 89.5822) (width 0.2) (layer "F.Cu") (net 9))
 (via (at 55.396155 93.10625) (size 0.6) (drill 0.3) (layers "F.Cu" "B.Cu") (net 9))
 (via (at 57.90625 73.38125) (size 0.6) (drill 0.3) (layers "F.Cu" "B.Cu") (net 9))
 (segment (start 57.90625 73.38125) (end 57.90625 74.474943) (width 0.2) (layer "B.Cu") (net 9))
 (segment (start 57.43685 93.901) (end 56.190905 93.901) (width 0.2) (layer "B.Cu") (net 9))
 (segment (start 58.1875 92.18125) (end 58.1875 93.15035) (width 0.2) (layer "B.Cu") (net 9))
 (segment (start 57.90625 74.474943) (end 58.6875 75.256193) (width 0.2) (layer "B.Cu") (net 9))
 (segment (start 58.6875 75.256193) (end 58.6875 77.81875) (width 0.2) (layer "B.Cu") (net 9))
 (segment (start 58.1875 93.15035) (end 57.43685 93.901) (width 0.2) (layer "B.Cu") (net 9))
 (segment (start 56.190905 93.901) (end 55.396155 93.10625) (width 0.2) (layer "B.Cu") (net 9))
 (segment (start 54.74 90.35) (end 52.96 90.35) (width 0.2) (layer "F.Cu") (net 14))
 (segment (start 57.375 74.375) (end 59.11875 74.375) (width 0.2) (layer "F.Cu") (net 6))
 (segment (start 55.25 78.09375) (end 55.25 78.025) (width 0.2) (layer "F.Cu") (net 6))
 (segment (start 55.11975 78.224) (end 55.25 78.09375) (width 0.2) (layer "F.Cu") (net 6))
 (segment (start 51.0329 92.50625) (end 47.94275 89.4161) (width 0.2) (layer "F.Cu") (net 6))
 (segment (start 47.94275 89.4161) (end 47.94275 80.5839) (width 0.2) (layer "F.Cu") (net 6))
 (segment (start 55.746812 92.50625) (end 51.0329 92.50625) (width 0.2) (layer "F.Cu") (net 6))
 (segment (start 47.94275 80.5839) (end 50.30265 78.224) (width 0.2) (layer "F.Cu") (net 6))
 (segment (start 59.11875 74.375) (end 59.1875 74.44375) (width 0.2) (layer "F.Cu") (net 6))
 (segment (start 55.25 76.5) (end 57.375 74.375) (width 0.2) (layer "F.Cu") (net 6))
 (segment (start 55.25 78.025) (end 55.25 76.5) (width 0.2) (layer "F.Cu") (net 6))
 (segment (start 50.30265 78.224) (end 55.11975 78.224) (width 0.2) (layer "F.Cu") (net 6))
 (segment (start 56.260906 93.020344) (end 55.746812 92.50625) (width 0.2) (layer "F.Cu") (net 6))
 (via (at 59.1875 74.44375) (size 0.6) (drill 0.3) (layers "F.Cu" "B.Cu") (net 6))
 (via (at 56.260906 93.020344) (size 0.6) (drill 0.3) (layers "F.Cu" "B.Cu") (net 6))
 (via (at 55.25 78.025) (size 0.6) (drill 0.3) (layers "F.Cu" "B.Cu") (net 6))
 (segment (start 59.1875 74.44375) (end 59.1875 77.81875) (width 0.2) (layer "B.Cu") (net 6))
 (segment (start 55.63 79.65) (end 55.63 78.405) (width 0.2) (layer "B.Cu") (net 6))
 (segment (start 55.63 78.405) (end 55.25 78.025) (width 0.2) (layer "B.Cu") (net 6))
 (segment (start 57.27075 93.5) (end 57.6875 93.08325) (width 0.2) (layer "B.Cu") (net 6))
 (segment (start 57.6875 93.08325) (end 57.6875 92.18125) (width 0.2) (layer "B.Cu") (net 6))
 (segment (start 56.740562 93.5) (end 57.27075 93.5) (width 0.2) (layer "B.Cu") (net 6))
 (segment (start 56.260906 93.020344) (end 56.740562 93.5) (width 0.2) (layer "B.Cu") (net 6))
 (segment (start 53.65625 77.5625) (end 53.65625 74.375) (width 0.2) (layer "F.Cu") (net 5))
 (segment (start 50.8997 93.50725) (end 54.726 93.50725) (width 0.2) (layer "F.Cu") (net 5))
 (segment (start 46.94175 79.15625) (end 46.94175 79.348) (width 0.2) (layer "F.Cu") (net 5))
 (segment (start 53.65625 74.375) (end 54.1875 73.84375) (width 0.2) (layer "F.Cu") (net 5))
 (segment (start 55.71975 94.501) (end 56.84375 94.501) (width 0.2) (layer "F.Cu") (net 5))
 (segment (start 54.726 93.50725) (end 55.71975 94.501) (width 0.2) (layer "F.Cu") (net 5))
 (segment (start 47.14075 89.7483) (end 50.8997 93.50725) (width 0.2) (layer "F.Cu") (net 5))
 (segment (start 46.94175 79.348) (end 47.14075 79.547) (width 0.2) (layer "F.Cu") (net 5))
 (segment (start 54.1875 73.84375) (end 56.84375 73.84375) (width 0.2) (layer "F.Cu") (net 5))
 (segment (start 47.14075 79.547) (end 47.14075 89.7483) (width 0.2) (layer "F.Cu") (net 5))
 (via (at 46.94175 79.15625) (size 0.6) (drill 0.3) (layers "F.Cu" "B.Cu") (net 5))
 (via (at 56.84375 94.501) (size 0.6) (drill 0.3) (layers "F.Cu" "B.Cu") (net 5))
 (via (at 56.84375 73.84375) (size 0.6) (drill 0.3) (layers "F.Cu" "B.Cu") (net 5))
 (via (at 53.65625 77.5625) (size 0.6) (drill 0.3) (layers "F.Cu" "B.Cu") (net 5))
 (segment (start 46.94175 79.15625) (end 48.5355 77.5625) (width 0.2) (layer "B.Cu") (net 5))
 (segment (start 53.65625 79.45625) (end 53.85 79.65) (width 0.2) (layer "B.Cu") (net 5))
 (segment (start 58.6875 93.230842) (end 58.6875 92.18125) (width 0.2) (layer "B.Cu") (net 5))
 (segment (start 53.65625 77.5625) (end 53.65625 79.45625) (width 0.2) (layer "B.Cu") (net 5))
 (segment (start 56.84375 73.84375) (end 56.84375 74.375) (width 0.2) (layer "B.Cu") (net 5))
 (segment (start 58.1875 75.71875) (end 58.1875 77.81875) (width 0.2) (layer "B.Cu") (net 5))
 (segment (start 48.5355 77.5625) (end 50.54989 77.5625) (width 0.2) (layer "B.Cu") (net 5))
 (segment (start 50.54989 77.5625) (end 51.58839 76.524) (width 0.2) (layer "B.Cu") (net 5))
 (segment (start 56.84375 94.501) (end 57.417342 94.501) (width 0.2) (layer "B.Cu") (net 5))
 (segment (start 57.417342 94.501) (end 58.6875 93.230842) (width 0.2) (layer "B.Cu") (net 5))
 (segment (start 51.58839 76.524) (end 52.61775 76.524) (width 0.2) (layer "B.Cu") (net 5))
 (segment (start 56.84375 74.375) (end 58.1875 75.71875) (width 0.2) (layer "B.Cu") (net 5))
 (segment (start 52.61775 76.524) (end 53.65625 77.5625) (width 0.2) (layer "B.Cu") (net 5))
 (segment (start 50.46875 78.625) (end 48.34375 80.75) (width 0.2) (layer "F.Cu") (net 8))
 (segment (start 48.34375 80.75) (end 48.34375 89.25) (width 0.2) (layer "F.Cu") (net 8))
 (segment (start 58.165 78.625) (end 50.46875 78.625) (width 0.2) (layer "F.Cu") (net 8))
 (segment (start 48.34375 89.25) (end 51 91.90625) (width 0.2) (layer "F.Cu") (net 8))
 (segment (start 51 91.90625) (end 56.3125 91.90625) (width 0.2) (layer "F.Cu") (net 8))
 (segment (start 59.19 79.65) (end 58.165 78.625) (width 0.2) (layer "F.Cu") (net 8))
 (via (at 56.3125 91.90625) (size 0.6) (drill 0.3) (layers "F.Cu" "B.Cu") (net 8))
 (segment (start 59.6875 79.1525) (end 59.6875 77.81875) (width 0.2) (layer "B.Cu") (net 8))
 (segment (start 56.3125 91.90625) (end 56.9125 91.90625) (width 0.2) (layer "B.Cu") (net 8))
 (segment (start 59.19 79.65) (end 59.6875 79.1525) (width 0.2) (layer "B.Cu") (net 8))
 (segment (start 56.9125 91.90625) (end 57.1875 92.18125) (width 0.2) (layer "B.Cu") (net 8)))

